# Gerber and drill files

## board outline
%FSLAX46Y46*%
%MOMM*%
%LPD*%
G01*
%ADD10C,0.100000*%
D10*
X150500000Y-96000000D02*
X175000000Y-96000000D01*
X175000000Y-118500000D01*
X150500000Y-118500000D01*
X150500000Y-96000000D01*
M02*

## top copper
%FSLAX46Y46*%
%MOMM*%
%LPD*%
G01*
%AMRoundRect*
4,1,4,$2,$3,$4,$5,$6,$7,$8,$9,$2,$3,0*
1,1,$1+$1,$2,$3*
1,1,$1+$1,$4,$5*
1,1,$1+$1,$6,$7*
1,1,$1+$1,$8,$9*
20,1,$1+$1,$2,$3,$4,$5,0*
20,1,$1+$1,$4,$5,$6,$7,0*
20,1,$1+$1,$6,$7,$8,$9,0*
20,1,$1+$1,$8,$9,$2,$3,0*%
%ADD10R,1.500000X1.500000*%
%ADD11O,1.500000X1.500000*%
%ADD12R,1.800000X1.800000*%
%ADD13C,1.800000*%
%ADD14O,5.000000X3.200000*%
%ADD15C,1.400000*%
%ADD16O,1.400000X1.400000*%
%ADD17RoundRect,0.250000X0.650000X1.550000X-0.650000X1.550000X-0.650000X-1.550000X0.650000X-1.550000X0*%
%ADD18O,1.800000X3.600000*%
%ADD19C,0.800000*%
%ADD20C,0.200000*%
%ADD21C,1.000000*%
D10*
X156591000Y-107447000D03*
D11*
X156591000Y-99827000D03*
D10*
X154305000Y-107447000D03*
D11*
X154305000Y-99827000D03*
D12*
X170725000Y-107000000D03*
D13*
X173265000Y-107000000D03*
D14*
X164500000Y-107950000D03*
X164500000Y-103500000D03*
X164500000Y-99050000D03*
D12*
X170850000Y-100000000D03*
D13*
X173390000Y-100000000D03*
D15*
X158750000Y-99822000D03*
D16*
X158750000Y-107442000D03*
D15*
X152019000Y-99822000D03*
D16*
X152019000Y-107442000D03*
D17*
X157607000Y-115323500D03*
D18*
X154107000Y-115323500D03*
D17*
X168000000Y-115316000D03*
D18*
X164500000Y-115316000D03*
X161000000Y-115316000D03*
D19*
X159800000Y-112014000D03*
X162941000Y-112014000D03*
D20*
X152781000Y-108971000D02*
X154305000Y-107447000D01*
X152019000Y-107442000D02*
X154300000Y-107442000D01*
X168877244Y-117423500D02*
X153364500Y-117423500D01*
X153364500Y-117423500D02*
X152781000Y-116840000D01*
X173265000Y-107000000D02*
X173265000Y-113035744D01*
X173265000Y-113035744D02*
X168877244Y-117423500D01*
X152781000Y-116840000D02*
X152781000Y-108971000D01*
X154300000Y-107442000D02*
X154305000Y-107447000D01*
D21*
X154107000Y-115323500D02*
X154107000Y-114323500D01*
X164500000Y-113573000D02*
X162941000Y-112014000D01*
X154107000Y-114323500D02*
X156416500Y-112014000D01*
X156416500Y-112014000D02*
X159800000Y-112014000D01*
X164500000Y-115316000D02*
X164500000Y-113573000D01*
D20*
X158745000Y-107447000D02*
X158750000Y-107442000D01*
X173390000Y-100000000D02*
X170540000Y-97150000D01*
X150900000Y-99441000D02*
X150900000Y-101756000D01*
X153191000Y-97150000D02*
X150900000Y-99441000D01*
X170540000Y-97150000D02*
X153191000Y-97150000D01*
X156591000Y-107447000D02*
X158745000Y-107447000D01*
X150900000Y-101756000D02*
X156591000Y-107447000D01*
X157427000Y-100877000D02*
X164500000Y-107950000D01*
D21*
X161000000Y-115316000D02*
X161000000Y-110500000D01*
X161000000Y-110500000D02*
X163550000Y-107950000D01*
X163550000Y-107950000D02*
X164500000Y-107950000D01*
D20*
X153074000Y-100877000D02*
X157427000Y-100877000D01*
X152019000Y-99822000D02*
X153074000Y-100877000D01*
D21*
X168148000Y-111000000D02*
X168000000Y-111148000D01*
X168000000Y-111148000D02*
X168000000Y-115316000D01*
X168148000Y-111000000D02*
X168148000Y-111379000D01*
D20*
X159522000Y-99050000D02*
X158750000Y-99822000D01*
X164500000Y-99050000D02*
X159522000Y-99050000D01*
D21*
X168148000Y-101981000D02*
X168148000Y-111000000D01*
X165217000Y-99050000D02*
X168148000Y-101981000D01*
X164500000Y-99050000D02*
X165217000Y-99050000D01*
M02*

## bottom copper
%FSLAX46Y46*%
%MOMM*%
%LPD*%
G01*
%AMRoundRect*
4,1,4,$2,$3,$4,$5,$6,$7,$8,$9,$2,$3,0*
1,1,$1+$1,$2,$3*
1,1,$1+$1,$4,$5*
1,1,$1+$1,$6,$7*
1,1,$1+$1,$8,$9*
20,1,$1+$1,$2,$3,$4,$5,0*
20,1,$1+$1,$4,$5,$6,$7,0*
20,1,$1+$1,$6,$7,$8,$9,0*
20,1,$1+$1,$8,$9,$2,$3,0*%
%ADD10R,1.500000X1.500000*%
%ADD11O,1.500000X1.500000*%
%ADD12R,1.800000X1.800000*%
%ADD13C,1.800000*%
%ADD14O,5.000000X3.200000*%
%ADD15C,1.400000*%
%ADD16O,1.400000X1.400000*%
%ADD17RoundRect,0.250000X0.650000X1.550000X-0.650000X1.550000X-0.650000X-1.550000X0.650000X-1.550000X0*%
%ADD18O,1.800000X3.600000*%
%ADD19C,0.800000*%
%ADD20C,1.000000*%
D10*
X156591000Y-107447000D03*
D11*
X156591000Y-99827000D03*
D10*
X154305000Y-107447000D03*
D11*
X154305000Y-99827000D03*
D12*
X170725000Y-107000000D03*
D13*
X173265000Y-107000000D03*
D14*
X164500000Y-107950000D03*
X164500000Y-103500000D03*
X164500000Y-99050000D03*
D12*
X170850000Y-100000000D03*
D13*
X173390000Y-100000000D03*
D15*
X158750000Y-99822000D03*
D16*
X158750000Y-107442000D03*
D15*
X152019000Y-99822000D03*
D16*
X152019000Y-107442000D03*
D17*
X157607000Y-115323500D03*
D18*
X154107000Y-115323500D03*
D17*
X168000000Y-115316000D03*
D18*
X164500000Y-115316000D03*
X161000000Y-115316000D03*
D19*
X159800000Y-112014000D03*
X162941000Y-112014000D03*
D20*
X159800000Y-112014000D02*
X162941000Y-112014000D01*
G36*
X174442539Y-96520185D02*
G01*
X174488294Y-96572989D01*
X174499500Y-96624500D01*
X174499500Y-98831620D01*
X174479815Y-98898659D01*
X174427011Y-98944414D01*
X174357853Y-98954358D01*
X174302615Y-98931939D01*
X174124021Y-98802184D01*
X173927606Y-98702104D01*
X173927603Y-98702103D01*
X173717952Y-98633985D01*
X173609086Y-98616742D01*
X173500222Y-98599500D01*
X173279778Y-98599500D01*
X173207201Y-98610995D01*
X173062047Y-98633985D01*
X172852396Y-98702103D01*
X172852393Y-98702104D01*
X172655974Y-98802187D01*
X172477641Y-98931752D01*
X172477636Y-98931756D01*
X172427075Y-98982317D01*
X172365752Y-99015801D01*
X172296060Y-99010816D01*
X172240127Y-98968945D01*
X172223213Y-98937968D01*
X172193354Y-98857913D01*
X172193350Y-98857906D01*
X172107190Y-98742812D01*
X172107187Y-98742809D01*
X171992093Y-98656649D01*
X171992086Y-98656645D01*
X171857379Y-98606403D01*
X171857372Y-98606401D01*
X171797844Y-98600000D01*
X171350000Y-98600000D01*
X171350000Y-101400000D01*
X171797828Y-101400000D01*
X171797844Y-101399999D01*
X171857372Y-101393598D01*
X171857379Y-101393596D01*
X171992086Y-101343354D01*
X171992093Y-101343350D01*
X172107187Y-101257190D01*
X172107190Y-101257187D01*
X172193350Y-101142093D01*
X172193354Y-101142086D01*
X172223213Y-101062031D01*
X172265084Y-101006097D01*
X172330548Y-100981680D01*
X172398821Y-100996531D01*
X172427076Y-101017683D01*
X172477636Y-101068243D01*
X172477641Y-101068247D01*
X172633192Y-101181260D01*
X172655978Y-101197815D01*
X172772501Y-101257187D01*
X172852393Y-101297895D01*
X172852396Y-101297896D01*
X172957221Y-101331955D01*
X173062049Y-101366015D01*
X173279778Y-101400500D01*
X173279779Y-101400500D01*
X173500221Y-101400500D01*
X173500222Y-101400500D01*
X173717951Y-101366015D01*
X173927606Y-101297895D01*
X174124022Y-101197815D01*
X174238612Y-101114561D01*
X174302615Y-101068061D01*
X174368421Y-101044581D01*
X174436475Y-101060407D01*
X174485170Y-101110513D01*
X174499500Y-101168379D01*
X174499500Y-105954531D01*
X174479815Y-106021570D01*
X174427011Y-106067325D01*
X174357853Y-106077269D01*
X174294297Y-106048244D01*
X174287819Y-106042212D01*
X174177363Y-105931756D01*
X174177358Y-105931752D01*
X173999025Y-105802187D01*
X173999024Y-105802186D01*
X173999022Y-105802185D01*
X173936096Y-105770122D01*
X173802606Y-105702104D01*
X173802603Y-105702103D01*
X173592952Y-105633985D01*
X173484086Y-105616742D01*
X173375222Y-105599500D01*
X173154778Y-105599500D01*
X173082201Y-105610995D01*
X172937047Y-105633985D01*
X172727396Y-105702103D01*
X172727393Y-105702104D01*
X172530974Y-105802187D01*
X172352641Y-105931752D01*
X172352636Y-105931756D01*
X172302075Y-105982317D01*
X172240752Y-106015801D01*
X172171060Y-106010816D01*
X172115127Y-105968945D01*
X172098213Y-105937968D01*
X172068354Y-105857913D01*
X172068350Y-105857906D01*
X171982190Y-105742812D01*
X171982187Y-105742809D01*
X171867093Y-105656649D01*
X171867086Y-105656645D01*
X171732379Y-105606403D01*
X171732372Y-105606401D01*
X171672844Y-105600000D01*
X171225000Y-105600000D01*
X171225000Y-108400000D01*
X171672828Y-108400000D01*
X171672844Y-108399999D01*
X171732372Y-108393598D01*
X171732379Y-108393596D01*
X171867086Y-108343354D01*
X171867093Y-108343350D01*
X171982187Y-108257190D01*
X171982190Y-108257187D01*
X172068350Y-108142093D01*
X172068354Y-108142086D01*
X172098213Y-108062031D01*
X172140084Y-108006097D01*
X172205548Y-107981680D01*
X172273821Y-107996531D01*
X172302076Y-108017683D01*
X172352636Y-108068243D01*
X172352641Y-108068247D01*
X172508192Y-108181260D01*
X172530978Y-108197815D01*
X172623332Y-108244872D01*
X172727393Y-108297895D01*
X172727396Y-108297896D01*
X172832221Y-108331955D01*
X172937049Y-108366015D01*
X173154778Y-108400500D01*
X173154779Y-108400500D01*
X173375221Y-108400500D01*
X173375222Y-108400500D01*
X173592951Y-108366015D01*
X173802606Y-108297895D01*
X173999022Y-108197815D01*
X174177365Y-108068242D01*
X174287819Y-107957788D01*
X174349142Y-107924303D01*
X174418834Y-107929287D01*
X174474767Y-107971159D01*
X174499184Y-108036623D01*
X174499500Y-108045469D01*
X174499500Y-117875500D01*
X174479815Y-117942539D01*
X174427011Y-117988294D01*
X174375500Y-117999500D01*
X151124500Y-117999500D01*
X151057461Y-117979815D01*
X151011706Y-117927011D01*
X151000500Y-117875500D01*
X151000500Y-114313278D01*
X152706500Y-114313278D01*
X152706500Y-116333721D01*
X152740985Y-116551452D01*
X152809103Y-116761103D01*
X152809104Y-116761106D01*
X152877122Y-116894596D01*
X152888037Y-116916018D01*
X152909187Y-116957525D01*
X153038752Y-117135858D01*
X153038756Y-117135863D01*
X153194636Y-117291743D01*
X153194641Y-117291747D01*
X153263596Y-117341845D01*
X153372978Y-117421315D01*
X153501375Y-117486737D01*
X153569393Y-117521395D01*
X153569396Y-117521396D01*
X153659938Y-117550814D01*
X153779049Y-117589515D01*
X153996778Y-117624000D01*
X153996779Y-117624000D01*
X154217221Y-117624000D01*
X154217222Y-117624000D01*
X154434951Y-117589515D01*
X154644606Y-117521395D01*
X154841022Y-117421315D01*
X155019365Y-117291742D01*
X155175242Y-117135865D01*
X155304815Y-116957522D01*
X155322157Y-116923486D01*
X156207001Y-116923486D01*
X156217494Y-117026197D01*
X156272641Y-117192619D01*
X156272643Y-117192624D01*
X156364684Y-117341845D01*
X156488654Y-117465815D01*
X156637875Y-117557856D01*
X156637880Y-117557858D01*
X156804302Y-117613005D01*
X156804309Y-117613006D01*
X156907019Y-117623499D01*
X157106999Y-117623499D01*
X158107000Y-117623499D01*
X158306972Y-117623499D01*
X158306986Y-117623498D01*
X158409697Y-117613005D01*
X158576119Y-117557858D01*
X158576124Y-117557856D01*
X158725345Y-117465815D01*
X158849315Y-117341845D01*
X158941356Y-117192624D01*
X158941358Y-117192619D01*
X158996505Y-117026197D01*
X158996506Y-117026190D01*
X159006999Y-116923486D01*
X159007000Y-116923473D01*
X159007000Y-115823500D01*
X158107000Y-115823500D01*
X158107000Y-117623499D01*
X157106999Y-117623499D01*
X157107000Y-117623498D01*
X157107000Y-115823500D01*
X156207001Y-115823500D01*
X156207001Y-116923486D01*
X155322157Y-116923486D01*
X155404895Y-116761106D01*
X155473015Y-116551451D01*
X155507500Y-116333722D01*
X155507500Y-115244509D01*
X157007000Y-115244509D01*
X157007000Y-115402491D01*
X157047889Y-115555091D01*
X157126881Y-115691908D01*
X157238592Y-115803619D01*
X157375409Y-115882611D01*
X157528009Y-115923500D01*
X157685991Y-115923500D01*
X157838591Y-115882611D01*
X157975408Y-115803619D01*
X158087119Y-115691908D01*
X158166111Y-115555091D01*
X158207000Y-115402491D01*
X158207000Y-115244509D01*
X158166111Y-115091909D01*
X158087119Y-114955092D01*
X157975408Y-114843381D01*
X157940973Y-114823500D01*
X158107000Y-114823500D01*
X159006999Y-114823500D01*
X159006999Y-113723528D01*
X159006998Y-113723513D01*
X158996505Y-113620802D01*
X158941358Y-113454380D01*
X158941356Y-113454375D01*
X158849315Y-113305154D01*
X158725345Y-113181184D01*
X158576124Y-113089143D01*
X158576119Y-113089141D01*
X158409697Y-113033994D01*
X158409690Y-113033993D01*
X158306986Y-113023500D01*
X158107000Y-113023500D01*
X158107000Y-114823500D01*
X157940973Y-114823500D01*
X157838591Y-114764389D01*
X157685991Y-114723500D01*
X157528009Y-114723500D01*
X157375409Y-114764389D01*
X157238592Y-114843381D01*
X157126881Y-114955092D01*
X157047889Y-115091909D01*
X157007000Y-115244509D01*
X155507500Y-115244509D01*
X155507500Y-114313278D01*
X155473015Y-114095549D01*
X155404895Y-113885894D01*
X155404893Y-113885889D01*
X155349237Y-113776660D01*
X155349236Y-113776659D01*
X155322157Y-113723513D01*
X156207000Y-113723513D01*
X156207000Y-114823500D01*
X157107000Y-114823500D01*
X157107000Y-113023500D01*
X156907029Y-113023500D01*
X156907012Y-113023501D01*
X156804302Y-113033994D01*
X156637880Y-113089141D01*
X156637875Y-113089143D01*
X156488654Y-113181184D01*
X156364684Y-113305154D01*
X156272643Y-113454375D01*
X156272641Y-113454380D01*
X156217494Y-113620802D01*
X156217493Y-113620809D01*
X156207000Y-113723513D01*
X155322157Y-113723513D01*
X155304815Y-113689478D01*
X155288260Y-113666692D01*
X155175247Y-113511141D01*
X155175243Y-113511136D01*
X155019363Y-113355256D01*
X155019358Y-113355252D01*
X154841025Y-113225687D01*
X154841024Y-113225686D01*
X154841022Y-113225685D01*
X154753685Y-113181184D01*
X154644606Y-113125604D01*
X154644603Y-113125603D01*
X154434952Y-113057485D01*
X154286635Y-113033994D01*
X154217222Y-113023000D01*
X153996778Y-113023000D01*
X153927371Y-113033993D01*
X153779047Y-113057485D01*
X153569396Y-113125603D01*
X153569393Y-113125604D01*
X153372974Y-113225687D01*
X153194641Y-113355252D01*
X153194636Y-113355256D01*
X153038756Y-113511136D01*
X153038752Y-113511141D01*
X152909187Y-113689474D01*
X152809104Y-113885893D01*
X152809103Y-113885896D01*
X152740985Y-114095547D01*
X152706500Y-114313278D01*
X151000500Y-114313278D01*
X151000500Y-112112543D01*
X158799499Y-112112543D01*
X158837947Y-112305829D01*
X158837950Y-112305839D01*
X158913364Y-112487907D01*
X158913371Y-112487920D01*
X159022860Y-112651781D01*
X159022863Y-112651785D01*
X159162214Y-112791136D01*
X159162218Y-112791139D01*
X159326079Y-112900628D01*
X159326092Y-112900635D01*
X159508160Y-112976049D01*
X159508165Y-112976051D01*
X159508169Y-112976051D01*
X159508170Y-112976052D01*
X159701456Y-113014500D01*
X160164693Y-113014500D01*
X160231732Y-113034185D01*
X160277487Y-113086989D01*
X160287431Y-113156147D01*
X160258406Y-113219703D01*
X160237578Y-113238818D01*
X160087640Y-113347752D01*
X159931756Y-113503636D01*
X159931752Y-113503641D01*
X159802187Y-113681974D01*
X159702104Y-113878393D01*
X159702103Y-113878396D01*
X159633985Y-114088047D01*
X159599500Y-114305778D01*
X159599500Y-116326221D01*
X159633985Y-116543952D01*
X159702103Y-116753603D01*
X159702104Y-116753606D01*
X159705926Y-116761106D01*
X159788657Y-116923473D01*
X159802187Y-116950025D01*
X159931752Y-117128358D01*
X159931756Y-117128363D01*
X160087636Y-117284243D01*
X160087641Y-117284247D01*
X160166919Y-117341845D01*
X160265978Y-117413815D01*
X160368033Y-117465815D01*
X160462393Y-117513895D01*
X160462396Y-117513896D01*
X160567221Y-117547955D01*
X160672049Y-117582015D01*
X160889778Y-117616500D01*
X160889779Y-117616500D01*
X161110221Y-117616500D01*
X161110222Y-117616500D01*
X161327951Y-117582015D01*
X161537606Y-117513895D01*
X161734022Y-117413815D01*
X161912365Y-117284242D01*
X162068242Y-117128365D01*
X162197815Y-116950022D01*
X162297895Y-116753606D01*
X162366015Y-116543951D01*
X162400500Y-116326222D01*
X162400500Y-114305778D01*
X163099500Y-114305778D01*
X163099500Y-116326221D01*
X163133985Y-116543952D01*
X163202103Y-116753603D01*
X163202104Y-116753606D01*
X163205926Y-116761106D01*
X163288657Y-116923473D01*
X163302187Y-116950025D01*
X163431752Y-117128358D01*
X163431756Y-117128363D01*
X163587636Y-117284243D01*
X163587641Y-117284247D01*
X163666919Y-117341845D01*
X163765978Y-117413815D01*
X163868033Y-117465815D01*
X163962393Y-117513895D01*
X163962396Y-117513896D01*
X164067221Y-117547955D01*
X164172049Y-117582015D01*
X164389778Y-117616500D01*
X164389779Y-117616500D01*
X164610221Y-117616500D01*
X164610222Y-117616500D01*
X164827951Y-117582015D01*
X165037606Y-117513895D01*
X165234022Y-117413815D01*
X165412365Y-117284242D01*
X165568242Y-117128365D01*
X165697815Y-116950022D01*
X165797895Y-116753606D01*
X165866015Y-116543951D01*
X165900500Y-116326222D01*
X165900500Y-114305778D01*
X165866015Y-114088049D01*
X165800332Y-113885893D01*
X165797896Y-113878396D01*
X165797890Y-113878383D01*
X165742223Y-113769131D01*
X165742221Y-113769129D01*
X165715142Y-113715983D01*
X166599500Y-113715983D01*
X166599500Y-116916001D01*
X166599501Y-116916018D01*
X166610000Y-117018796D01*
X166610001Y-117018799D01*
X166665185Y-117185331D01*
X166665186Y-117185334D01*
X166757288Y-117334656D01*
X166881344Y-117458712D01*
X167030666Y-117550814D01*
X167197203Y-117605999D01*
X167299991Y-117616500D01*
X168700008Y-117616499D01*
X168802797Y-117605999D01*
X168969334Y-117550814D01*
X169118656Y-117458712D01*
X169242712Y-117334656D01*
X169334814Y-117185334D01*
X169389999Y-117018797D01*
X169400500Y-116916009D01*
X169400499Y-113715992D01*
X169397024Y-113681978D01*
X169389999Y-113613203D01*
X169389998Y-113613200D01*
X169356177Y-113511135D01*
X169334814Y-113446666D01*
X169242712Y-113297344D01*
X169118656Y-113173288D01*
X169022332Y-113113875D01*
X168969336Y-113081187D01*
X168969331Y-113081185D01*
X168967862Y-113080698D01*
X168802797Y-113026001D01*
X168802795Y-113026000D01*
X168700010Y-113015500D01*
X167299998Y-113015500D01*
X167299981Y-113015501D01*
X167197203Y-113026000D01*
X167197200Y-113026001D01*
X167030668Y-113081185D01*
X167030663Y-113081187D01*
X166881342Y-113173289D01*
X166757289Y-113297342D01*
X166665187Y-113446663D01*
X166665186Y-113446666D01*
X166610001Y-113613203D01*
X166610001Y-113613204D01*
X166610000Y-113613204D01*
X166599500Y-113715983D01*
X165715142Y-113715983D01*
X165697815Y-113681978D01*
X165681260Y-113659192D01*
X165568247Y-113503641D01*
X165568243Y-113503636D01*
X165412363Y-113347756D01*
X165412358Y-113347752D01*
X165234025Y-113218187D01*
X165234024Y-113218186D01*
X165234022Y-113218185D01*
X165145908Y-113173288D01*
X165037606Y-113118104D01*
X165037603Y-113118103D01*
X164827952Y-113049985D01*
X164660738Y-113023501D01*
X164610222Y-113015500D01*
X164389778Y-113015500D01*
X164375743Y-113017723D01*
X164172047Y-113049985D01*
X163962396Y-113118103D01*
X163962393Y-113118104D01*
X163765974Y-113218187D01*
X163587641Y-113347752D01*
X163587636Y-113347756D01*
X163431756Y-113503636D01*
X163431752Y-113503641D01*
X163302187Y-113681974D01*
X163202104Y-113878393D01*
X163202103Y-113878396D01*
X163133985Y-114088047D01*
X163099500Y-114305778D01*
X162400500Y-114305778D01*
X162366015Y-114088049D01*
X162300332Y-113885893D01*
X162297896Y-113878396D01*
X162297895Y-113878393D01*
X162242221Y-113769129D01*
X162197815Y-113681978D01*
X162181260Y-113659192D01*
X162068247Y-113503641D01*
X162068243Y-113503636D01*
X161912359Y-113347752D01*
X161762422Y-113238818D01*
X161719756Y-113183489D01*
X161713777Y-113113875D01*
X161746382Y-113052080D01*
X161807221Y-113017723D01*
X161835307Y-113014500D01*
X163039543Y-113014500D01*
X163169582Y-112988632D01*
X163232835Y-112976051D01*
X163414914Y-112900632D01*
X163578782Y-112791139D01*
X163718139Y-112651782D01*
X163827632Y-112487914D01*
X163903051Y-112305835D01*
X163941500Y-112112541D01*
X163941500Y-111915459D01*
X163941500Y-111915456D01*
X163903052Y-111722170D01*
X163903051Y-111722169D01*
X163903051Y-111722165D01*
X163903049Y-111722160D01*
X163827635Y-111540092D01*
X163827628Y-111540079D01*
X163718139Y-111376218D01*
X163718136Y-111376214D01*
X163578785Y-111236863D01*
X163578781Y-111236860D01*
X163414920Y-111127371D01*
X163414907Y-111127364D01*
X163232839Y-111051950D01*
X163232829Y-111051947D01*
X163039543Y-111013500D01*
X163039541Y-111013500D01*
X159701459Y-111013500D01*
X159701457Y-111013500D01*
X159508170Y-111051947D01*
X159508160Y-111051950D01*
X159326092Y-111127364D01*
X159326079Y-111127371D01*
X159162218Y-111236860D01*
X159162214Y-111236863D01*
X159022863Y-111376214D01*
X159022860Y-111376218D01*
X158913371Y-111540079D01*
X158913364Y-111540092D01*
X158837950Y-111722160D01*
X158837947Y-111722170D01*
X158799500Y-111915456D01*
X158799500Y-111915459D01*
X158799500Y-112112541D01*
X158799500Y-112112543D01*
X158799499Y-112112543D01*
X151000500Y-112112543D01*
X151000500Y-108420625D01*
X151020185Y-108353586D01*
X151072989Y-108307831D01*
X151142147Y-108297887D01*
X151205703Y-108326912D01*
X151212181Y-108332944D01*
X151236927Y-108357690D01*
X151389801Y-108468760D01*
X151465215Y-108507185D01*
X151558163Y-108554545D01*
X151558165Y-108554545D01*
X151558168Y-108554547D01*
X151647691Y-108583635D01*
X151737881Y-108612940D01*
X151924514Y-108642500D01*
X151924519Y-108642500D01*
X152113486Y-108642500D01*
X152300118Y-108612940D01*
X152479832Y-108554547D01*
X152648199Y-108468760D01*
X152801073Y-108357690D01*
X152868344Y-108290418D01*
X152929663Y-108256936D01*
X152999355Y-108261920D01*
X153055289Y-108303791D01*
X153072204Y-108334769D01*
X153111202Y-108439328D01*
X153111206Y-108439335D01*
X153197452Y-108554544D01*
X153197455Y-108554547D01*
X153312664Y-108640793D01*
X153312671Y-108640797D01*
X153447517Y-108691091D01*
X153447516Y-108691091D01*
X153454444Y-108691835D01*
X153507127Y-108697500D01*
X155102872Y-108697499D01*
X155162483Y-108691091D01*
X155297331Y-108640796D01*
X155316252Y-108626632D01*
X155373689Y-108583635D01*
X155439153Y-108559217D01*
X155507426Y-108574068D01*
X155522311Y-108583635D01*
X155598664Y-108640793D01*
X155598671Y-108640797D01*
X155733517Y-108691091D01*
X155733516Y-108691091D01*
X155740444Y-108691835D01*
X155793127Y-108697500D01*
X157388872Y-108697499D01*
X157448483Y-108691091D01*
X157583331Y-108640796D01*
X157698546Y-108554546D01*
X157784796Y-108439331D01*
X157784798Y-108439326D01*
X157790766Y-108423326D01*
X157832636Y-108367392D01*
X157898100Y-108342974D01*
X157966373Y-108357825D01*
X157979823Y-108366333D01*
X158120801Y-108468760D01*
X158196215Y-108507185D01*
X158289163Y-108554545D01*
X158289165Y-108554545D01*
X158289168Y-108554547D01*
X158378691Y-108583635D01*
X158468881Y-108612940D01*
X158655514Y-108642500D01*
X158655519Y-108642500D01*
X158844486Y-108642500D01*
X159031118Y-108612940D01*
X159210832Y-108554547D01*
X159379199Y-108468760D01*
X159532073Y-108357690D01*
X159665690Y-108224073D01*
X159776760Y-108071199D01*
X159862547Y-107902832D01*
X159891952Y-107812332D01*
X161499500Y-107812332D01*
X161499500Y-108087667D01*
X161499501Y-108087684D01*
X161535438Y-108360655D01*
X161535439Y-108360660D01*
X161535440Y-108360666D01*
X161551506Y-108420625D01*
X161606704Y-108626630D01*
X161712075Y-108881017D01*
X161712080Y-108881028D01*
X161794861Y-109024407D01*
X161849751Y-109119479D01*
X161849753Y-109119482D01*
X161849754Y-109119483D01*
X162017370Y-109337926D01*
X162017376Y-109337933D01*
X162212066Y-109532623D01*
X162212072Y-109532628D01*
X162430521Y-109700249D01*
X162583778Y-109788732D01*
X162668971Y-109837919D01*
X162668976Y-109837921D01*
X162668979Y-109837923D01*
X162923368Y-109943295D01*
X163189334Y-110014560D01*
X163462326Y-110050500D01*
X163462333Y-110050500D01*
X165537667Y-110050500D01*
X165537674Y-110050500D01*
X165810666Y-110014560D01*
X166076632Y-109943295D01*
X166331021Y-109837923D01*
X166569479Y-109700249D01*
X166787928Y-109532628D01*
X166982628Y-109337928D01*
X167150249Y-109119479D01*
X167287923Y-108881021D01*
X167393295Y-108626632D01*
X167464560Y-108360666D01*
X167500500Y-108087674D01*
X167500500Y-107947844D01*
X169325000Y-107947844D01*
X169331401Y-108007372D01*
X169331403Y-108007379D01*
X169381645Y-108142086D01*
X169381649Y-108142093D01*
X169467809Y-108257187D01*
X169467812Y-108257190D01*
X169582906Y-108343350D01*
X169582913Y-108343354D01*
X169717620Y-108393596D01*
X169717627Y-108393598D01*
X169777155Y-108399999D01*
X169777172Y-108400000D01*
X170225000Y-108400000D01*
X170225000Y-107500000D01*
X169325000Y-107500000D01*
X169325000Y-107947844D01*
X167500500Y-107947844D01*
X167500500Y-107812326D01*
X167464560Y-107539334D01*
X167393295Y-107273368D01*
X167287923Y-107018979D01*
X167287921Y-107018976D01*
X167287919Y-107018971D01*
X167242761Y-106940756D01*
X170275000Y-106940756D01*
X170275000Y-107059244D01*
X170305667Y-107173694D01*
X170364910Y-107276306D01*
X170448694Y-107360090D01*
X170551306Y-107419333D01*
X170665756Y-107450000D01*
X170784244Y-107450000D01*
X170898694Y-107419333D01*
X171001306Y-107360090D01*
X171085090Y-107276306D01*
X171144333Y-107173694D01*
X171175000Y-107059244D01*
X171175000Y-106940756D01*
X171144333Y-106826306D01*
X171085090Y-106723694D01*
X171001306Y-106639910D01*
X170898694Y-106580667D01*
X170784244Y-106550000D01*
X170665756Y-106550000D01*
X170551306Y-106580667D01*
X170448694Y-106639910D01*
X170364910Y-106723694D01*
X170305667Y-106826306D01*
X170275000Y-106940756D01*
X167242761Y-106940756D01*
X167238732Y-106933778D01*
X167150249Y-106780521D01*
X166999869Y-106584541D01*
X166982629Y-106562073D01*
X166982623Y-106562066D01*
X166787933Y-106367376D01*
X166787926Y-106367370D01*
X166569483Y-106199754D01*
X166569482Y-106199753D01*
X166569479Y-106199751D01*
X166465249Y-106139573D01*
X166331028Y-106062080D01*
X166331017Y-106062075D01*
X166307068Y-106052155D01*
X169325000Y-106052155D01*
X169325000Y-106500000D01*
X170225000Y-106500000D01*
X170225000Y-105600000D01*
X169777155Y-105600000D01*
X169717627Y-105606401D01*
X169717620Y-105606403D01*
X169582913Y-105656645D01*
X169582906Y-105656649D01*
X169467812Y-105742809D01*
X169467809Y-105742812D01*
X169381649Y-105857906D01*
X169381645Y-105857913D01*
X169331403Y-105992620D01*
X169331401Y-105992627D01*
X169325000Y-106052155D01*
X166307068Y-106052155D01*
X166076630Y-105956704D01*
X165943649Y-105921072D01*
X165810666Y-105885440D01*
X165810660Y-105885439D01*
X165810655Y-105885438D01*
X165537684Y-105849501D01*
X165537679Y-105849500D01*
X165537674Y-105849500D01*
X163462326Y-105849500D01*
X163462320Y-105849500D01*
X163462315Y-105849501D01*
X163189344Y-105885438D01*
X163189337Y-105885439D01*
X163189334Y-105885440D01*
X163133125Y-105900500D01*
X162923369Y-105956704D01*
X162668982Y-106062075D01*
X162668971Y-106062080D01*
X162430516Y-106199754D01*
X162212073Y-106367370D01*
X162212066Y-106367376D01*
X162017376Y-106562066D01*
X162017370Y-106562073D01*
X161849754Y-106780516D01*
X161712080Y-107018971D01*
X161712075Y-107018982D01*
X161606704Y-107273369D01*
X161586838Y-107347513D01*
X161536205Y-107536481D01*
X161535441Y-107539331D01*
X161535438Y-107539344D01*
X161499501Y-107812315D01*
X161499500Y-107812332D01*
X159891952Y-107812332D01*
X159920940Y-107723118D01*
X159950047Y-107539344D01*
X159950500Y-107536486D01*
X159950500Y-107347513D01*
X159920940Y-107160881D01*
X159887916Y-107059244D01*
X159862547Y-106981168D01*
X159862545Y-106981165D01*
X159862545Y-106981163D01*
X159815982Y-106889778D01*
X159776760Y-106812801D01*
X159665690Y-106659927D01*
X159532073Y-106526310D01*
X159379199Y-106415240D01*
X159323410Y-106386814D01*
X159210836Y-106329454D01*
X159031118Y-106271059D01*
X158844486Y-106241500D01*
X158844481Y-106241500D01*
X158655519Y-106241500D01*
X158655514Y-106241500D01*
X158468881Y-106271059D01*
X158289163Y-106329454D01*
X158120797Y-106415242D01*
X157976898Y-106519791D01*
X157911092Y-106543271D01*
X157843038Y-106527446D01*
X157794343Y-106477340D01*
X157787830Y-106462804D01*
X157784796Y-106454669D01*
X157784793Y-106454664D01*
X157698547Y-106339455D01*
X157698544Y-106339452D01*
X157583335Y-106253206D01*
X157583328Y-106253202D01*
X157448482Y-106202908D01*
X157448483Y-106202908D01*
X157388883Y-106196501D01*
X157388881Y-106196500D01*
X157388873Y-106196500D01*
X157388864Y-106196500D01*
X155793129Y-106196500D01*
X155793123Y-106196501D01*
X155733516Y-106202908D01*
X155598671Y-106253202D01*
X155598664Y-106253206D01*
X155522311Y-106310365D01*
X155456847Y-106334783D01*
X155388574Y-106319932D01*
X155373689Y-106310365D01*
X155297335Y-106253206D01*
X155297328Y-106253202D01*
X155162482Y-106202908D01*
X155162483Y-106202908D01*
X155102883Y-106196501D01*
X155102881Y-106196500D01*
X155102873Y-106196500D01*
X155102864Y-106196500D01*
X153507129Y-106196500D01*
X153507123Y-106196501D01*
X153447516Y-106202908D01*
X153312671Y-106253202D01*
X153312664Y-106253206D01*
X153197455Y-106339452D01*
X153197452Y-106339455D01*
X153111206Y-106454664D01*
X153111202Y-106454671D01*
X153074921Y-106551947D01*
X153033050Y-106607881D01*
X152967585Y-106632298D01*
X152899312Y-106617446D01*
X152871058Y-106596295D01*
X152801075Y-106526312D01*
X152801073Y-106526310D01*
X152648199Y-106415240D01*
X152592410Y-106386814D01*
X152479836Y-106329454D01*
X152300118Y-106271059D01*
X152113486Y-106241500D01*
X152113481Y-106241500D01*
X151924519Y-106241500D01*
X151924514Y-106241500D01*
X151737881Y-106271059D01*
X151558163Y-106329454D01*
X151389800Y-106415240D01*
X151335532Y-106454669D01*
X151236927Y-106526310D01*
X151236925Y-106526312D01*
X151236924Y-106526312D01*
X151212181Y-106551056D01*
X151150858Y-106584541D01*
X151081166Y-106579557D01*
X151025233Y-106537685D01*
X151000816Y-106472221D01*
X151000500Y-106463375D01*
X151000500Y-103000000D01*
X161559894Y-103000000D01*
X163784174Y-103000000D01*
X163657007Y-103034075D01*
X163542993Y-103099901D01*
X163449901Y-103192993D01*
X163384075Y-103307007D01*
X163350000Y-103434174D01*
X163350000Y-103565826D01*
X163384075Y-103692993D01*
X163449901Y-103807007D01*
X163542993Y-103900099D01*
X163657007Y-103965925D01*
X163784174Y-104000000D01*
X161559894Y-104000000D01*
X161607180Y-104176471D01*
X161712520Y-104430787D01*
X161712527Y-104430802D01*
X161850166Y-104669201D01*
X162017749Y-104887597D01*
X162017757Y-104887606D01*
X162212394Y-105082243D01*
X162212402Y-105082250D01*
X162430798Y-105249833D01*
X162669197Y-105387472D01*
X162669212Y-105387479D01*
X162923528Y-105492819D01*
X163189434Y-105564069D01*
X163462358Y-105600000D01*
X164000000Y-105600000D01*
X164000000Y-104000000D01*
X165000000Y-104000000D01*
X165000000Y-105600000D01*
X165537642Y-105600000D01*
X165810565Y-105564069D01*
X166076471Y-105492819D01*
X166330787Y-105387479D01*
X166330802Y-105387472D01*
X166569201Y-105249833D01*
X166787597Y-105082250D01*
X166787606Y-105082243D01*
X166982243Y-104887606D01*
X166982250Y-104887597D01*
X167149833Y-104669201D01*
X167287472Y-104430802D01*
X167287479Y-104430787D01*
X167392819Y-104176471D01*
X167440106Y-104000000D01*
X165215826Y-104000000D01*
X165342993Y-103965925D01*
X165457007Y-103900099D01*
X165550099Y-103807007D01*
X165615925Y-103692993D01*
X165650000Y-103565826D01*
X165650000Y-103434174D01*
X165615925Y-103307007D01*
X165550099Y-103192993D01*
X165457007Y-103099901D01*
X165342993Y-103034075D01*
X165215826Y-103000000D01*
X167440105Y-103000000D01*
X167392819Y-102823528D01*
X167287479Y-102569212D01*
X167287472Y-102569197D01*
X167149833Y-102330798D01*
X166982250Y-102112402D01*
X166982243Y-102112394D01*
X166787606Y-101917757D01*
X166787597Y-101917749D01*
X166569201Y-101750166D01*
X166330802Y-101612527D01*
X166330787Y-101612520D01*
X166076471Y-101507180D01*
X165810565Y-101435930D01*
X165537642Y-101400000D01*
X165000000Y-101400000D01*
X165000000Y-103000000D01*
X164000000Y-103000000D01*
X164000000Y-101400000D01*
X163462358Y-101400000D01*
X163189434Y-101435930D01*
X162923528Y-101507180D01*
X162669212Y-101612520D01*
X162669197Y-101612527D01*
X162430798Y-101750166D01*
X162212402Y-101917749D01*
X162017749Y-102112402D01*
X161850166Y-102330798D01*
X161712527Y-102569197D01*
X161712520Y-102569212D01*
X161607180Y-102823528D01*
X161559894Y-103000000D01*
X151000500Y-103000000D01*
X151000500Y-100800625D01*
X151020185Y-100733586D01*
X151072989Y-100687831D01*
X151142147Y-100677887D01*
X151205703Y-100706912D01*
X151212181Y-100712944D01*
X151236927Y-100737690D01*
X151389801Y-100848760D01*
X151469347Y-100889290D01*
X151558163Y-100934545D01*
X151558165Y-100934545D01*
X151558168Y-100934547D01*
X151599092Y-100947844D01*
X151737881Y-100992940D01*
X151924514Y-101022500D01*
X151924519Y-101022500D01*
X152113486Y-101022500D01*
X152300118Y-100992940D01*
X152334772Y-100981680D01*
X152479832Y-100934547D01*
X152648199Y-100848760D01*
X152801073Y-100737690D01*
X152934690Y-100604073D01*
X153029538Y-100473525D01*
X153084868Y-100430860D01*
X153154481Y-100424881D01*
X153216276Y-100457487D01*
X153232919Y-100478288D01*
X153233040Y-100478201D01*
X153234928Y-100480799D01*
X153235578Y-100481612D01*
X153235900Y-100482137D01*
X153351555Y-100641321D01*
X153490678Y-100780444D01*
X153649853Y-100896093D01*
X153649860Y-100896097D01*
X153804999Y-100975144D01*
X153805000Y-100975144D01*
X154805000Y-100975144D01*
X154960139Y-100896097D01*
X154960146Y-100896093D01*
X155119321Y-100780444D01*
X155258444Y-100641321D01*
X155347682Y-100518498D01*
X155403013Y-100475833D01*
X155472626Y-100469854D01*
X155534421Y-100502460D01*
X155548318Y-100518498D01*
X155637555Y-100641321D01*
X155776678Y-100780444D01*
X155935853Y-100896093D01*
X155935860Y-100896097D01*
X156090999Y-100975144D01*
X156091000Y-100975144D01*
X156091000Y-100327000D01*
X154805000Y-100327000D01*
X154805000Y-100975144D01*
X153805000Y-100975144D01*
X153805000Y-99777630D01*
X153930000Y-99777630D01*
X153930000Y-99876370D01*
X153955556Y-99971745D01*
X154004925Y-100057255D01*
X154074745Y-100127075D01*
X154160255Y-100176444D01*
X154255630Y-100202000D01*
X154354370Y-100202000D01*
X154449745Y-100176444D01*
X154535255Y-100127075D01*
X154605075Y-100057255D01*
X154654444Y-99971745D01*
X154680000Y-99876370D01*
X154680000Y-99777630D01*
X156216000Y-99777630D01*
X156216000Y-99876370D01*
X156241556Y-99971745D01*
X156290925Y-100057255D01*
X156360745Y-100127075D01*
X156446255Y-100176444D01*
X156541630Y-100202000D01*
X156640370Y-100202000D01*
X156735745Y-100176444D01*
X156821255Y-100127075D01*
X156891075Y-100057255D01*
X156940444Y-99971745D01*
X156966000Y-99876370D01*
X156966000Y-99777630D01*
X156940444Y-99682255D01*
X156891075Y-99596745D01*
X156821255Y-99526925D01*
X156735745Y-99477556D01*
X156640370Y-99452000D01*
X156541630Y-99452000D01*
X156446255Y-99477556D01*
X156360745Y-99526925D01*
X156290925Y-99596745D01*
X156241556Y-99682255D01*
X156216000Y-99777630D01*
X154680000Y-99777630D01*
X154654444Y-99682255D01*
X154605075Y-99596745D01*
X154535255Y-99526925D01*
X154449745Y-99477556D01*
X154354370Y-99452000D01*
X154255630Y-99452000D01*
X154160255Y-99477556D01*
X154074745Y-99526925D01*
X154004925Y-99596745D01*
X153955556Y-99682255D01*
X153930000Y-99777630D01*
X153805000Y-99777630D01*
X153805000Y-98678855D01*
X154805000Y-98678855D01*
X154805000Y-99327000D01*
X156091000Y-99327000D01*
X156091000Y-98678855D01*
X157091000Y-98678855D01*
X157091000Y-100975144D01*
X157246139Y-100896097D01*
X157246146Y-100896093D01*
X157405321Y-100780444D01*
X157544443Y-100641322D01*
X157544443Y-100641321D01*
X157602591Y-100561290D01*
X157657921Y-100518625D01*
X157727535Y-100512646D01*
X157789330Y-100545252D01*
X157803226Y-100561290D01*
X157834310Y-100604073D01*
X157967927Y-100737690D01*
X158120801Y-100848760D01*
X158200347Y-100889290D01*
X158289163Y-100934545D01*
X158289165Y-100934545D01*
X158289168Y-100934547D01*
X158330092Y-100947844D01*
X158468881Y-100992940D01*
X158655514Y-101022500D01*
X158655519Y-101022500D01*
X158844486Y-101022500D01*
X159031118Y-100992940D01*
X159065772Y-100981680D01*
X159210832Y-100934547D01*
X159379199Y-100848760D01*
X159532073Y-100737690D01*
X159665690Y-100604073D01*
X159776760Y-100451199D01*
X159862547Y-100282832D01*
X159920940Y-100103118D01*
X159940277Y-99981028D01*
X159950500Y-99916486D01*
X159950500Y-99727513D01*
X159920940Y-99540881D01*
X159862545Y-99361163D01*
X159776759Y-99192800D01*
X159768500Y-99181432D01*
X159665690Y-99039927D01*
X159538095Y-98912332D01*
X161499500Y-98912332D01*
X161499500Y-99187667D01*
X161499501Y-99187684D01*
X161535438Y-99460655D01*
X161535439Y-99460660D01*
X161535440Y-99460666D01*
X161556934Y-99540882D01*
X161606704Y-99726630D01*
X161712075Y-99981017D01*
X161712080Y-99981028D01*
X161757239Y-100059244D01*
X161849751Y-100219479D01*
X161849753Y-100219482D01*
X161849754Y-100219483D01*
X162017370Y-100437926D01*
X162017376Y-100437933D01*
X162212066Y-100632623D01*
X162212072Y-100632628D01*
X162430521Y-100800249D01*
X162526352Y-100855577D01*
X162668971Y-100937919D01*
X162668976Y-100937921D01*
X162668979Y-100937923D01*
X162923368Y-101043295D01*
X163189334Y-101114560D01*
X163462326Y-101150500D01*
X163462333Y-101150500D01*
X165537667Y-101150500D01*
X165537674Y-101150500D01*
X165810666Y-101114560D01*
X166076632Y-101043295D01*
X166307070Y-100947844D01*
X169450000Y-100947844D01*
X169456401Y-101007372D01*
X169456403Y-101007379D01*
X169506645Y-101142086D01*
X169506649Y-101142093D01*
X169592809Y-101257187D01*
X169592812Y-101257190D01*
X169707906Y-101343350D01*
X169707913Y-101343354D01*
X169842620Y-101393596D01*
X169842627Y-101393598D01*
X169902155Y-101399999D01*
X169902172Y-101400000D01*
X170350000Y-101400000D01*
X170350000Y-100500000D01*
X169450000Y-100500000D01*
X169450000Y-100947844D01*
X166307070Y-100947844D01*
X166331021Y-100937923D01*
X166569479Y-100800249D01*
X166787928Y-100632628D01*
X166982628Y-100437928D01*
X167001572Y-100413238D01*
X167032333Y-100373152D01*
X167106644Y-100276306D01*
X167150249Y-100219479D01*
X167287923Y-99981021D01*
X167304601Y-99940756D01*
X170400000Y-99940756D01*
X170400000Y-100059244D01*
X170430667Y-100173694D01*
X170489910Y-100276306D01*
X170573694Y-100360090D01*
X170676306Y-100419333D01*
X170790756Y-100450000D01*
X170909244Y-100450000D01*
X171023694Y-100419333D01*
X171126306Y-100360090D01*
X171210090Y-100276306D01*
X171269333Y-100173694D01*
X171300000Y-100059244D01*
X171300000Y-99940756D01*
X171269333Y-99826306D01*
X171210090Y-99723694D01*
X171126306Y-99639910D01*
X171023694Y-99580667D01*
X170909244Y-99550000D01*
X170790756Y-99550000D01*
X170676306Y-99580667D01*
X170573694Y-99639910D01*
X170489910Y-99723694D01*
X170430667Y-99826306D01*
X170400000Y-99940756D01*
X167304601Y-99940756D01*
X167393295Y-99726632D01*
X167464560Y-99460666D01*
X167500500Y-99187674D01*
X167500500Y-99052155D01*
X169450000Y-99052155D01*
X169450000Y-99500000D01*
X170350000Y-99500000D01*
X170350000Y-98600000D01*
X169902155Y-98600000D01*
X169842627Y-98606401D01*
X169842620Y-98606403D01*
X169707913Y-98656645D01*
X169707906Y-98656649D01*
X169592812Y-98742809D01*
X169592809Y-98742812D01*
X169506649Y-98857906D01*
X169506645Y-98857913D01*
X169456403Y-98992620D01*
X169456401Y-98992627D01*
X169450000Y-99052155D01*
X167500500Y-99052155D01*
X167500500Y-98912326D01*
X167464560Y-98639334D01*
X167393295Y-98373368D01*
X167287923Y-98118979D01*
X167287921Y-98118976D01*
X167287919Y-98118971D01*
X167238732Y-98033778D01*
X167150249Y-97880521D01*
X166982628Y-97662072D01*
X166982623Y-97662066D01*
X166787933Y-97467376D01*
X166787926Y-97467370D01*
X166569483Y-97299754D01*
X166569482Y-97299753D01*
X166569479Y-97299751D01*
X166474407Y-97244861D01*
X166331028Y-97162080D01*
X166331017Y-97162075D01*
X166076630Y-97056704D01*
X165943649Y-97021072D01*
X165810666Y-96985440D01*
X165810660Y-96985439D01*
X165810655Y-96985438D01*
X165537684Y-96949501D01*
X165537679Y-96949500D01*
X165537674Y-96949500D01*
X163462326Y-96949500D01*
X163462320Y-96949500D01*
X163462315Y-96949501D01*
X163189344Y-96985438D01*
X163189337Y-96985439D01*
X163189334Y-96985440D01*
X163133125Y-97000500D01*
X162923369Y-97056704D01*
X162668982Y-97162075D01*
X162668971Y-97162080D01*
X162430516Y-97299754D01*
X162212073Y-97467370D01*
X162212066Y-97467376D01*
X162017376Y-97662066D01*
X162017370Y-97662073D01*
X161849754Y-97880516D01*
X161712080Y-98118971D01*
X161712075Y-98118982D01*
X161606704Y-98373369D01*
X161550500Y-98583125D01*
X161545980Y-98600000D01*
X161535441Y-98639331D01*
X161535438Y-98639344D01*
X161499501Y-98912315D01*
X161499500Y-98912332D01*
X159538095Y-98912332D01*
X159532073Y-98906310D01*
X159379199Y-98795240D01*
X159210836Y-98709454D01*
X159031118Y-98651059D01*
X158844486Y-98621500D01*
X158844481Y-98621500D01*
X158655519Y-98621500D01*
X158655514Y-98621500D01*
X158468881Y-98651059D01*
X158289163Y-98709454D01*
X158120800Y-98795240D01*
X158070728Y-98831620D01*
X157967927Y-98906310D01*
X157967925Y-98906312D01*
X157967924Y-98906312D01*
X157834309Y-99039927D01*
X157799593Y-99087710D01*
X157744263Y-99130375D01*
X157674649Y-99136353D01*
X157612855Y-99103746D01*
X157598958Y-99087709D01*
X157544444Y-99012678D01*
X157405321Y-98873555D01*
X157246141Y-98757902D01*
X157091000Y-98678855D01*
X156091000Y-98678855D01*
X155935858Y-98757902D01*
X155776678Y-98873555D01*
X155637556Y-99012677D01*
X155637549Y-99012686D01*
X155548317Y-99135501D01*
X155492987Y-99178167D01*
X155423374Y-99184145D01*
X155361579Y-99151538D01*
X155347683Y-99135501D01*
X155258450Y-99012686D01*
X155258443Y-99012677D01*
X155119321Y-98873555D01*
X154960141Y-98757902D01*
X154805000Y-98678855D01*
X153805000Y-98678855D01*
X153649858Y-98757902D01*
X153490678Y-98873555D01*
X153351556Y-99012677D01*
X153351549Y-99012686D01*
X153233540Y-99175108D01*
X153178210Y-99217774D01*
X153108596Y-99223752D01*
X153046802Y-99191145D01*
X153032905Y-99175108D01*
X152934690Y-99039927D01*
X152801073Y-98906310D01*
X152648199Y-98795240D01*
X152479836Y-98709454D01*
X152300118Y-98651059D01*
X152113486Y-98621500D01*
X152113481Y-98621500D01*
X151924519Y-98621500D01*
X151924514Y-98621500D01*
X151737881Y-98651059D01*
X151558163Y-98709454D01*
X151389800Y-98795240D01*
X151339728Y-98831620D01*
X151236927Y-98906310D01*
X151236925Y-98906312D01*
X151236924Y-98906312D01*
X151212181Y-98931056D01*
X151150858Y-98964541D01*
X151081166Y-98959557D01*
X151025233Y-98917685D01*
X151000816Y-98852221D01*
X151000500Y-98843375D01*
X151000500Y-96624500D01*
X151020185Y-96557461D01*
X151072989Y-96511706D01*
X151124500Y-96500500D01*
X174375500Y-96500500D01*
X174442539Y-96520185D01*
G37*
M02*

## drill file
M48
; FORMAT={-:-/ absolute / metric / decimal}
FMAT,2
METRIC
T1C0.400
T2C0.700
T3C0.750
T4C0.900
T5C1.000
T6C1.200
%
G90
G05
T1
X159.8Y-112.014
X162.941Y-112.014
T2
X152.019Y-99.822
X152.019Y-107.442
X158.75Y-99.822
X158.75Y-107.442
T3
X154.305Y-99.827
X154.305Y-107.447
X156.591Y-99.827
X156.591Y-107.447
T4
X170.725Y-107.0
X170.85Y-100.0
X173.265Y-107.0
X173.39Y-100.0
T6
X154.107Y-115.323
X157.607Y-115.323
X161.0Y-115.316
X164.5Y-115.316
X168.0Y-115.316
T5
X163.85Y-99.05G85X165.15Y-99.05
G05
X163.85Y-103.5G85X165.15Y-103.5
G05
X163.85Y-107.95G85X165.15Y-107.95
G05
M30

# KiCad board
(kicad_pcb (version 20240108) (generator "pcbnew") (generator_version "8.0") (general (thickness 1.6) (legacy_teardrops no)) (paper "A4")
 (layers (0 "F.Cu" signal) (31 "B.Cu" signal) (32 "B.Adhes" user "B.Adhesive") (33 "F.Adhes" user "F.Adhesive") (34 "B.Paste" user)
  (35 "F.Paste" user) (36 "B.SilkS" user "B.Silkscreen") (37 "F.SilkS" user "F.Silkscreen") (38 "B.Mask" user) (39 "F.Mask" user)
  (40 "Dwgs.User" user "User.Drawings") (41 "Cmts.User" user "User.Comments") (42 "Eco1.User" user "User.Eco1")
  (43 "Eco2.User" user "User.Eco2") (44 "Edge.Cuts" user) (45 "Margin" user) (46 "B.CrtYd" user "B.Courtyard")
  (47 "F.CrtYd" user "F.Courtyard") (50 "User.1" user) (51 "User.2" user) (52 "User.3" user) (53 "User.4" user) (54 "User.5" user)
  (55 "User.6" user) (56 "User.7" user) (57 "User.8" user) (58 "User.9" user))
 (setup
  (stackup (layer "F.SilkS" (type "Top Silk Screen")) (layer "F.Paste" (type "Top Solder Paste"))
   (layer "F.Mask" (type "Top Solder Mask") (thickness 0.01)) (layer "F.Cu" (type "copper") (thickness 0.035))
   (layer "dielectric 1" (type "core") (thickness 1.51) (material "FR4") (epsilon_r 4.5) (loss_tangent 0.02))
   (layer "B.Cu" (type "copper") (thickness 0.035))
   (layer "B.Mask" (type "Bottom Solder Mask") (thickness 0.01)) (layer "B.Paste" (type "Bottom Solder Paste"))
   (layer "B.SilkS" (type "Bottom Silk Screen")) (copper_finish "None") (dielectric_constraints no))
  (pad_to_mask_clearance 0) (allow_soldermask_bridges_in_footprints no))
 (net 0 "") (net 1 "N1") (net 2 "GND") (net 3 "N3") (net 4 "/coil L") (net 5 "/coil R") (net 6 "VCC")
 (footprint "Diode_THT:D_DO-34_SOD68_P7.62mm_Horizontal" (layer "F.Cu") (at 156.591 107.447 90)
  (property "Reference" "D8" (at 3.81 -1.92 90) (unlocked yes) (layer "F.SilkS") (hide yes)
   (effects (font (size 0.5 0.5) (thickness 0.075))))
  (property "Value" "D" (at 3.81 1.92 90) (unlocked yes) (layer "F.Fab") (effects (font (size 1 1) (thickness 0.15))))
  (pad "1" thru_hole rect (at 0 0 90) (size 1.5 1.5) (drill 0.75) (layers "*.Cu" "*.Mask") (remove_unused_layers no) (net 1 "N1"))
  (pad "2" thru_hole oval (at 7.62 0 90) (size 1.5 1.5) (drill 0.75) (layers "*.Cu" "*.Mask") (remove_unused_layers no) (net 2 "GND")))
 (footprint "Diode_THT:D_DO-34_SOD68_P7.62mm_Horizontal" (layer "F.Cu") (at 154.305 107.447 90)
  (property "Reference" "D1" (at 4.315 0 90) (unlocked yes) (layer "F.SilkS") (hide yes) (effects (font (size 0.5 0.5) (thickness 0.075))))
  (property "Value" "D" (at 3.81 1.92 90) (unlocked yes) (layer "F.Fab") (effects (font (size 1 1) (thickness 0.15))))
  (pad "1" thru_hole rect (at 0 0 90) (size 1.5 1.5) (drill 0.75) (layers "*.Cu" "*.Mask") (remove_unused_layers no) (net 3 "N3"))
  (pad "2" thru_hole oval (at 7.62 0 90) (size 1.5 1.5) (drill 0.75) (layers "*.Cu" "*.Mask") (remove_unused_layers no) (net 2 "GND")))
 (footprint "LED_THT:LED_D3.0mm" (layer "F.Cu") (at 170.725 107)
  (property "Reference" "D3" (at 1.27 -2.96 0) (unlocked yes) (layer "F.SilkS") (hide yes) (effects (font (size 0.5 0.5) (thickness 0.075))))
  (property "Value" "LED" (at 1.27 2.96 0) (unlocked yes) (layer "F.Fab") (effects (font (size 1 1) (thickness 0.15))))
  (pad "1" thru_hole rect (at 0 0) (size 1.8 1.8) (drill 0.9) (layers "*.Cu" "*.Mask") (remove_unused_layers no) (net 2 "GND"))
  (pad "2" thru_hole circle (at 2.54 0) (size 1.8 1.8) (drill 0.9) (layers "*.Cu" "*.Mask") (remove_unused_layers no) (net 3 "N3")))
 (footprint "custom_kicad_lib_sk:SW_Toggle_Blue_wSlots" (layer "F.Cu") (at 164.5 103.5 90)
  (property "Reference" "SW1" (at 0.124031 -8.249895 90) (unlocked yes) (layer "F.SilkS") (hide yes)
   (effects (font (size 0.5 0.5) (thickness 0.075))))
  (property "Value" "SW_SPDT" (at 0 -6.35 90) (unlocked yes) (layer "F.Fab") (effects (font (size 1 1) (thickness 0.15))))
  (pad "1" thru_hole oval (at -4.45 0 90) (size 3.2 5) (drill oval 1 2.3) (layers "*.Cu" "*.Mask") (remove_unused_layers no)
   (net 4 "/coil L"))
  (pad "2" thru_hole oval (at 0 0 90) (size 3.2 5) (drill oval 1 2.3) (layers "*.Cu" "*.Mask") (remove_unused_layers no) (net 2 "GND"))
  (pad "3" thru_hole oval (at 4.45 0 90) (size 3.2 5) (drill oval 1 2.3) (layers "*.Cu" "*.Mask") (remove_unused_layers no)
   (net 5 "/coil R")))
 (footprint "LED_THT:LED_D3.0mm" (layer "F.Cu") (at 170.85 100)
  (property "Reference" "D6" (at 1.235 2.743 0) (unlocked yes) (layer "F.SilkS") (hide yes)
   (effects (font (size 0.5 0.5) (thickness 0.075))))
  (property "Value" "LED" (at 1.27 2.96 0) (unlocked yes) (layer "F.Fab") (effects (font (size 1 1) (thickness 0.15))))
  (pad "1" thru_hole rect (at 0 0) (size 1.8 1.8) (drill 0.9) (layers "*.Cu" "*.Mask") (remove_unused_layers no) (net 2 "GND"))
  (pad "2" thru_hole circle (at 2.54 0) (size 1.8 1.8) (drill 0.9) (layers "*.Cu" "*.Mask") (remove_unused_layers no) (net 1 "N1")))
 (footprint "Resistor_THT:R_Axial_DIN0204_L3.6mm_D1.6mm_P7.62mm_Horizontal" (layer "F.Cu") (at 158.75 99.822 -90)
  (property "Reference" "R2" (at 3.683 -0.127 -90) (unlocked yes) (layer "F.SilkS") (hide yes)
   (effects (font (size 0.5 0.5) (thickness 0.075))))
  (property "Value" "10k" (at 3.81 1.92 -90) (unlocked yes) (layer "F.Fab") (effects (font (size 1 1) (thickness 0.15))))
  (pad "1" thru_hole circle (at 0 0 270) (size 1.4 1.4) (drill 0.7) (layers "*.Cu" "*.Mask") (remove_unused_layers no) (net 5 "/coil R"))
  (pad "2" thru_hole oval (at 7.62 0 270) (size 1.4 1.4) (drill 0.7) (layers "*.Cu" "*.Mask") (remove_unused_layers no) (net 1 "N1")))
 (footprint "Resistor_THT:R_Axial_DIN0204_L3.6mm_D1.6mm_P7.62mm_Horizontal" (layer "F.Cu") (at 152.019 99.822 -90)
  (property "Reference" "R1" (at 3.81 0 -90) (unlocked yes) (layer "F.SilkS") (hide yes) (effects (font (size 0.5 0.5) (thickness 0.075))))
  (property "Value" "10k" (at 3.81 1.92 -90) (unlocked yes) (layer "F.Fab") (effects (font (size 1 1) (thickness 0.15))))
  (pad "1" thru_hole circle (at 0 0 270) (size 1.4 1.4) (drill 0.7) (layers "*.Cu" "*.Mask") (remove_unused_layers no) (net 4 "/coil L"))
  (pad "2" thru_hole oval (at 7.62 0 270) (size 1.4 1.4) (drill 0.7) (layers "*.Cu" "*.Mask") (remove_unused_layers no) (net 3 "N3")))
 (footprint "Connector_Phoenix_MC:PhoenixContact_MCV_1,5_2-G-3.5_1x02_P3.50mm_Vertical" (layer "B.Cu") (at 157.607 115.3235 180)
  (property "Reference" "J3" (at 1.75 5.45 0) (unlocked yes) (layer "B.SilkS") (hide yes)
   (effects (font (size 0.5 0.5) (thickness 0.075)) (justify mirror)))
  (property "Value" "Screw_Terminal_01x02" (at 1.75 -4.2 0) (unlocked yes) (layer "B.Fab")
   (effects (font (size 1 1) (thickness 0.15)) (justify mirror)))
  (pad "1" thru_hole roundrect (at 0 0 180) (size 1.8 3.6) (drill 1.2) (layers "*.Cu" "*.Mask") (remove_unused_layers no)
   (roundrect_rratio 0.138889) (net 2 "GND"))
  (pad "2" thru_hole oval (at 3.5 0 180) (size 1.8 3.6) (drill 1.2) (layers "*.Cu" "*.Mask") (remove_unused_layers no) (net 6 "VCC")))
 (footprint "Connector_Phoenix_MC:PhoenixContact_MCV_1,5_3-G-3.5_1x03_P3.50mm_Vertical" (layer "B.Cu") (at 168 115.316 180)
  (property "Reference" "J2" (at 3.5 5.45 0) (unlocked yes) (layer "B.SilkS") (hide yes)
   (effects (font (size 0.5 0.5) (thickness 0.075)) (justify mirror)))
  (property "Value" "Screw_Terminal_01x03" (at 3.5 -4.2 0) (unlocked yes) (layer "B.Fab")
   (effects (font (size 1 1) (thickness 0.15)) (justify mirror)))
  (pad "1" thru_hole roundrect (at 0 0 180) (size 1.8 3.6) (drill 1.2) (layers "*.Cu" "*.Mask") (remove_unused_layers no)
   (roundrect_rratio 0.138889) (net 5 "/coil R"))
  (pad "2" thru_hole oval (at 3.5 0 180) (size 1.8 3.6) (drill 1.2) (layers "*.Cu" "*.Mask") (remove_unused_layers no) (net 6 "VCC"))
  (pad "3" thru_hole oval (at 7 0 180) (size 1.8 3.6) (drill 1.2) (layers "*.Cu" "*.Mask") (remove_unused_layers no) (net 4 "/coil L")))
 (gr_rect (start 150.5 96) (end 175 118.5) (stroke (width 0.1) (type default)) (fill none) (layer "Edge.Cuts"))
 (segment (start 152.781 108.971) (end 154.305 107.447) (width 0.2) (layer "F.Cu") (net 3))
 (segment (start 152.019 107.442) (end 154.3 107.442) (width 0.2) (layer "F.Cu") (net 3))
 (segment (start 168.877244 117.4235) (end 153.3645 117.4235) (width 0.2) (layer "F.Cu") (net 3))
 (segment (start 153.3645 117.4235) (end 152.781 116.84) (width 0.2) (layer "F.Cu") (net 3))
 (segment (start 173.265 107) (end 173.265 113.035744) (width 0.2) (layer "F.Cu") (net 3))
 (segment (start 173.265 113.035744) (end 168.877244 117.4235) (width 0.2) (layer "F.Cu") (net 3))
 (segment (start 152.781 116.84) (end 152.781 108.971) (width 0.2) (layer "F.Cu") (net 3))
 (segment (start 154.3 107.442) (end 154.305 107.447) (width 0.2) (layer "F.Cu") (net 3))
 (segment (start 154.107 115.3235) (end 154.107 114.3235) (width 1) (layer "F.Cu") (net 6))
 (segment (start 164.5 113.573) (end 162.941 112.014) (width 1) (layer "F.Cu") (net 6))
 (segment (start 154.107 114.3235) (end 156.4165 112.014) (width 1) (layer "F.Cu") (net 6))
 (segment (start 156.4165 112.014) (end 159.8 112.014) (width 1) (layer "F.Cu") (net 6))
 (segment (start 164.5 115.316) (end 164.5 113.573) (width 1) (layer "F.Cu") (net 6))
 (via (at 159.8 112.014) (size 0.8) (drill 0.4) (layers "F.Cu" "B.Cu") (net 6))
 (via (at 162.941 112.014) (size 0.8) (drill 0.4) (layers "F.Cu" "B.Cu") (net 6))
 (segment (start 159.8 112.014) (end 162.941 112.014) (width 1) (layer "B.Cu") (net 6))
 (segment (start 158.745 107.447) (end 158.75 107.442) (width 0.2) (layer "F.Cu") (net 1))
 (segment (start 173.39 100) (end 170.54 97.15) (width 0.2) (layer "F.Cu") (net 1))
 (segment (start 150.9 99.441) (end 150.9 101.756) (width 0.2) (layer "F.Cu") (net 1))
 (segment (start 153.191 97.15) (end 150.9 99.441) (width 0.2) (layer "F.Cu") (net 1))
 (segment (start 170.54 97.15) (end 153.191 97.15) (width 0.2) (layer "F.Cu") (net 1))
 (segment (start 156.591 107.447) (end 158.745 107.447) (width 0.2) (layer "F.Cu") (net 1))
 (segment (start 150.9 101.756) (end 156.591 107.447) (width 0.2) (layer "F.Cu") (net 1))
 (segment (start 157.427 100.877) (end 164.5 107.95) (width 0.2) (layer "F.Cu") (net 4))
 (segment (start 161 115.316) (end 161 110.5) (width 1) (layer "F.Cu") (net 4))
 (segment (start 161 110.5) (end 163.55 107.95) (width 1) (layer "F.Cu") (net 4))
 (segment (start 163.55 107.95) (end 164.5 107.95) (width 1) (layer "F.Cu") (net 4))
 (segment (start 153.074 100.877) (end 157.427 100.877) (width 0.2) (layer "F.Cu") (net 4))
 (segment (start 152.019 99.822) (end 153.074 100.877) (width 0.2) (layer "F.Cu") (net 4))
 (segment (start 168.148 111) (end 168 111.148) (width 1) (layer "F.Cu") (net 5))
 (segment (start 168 111.148) (end 168 115.316) (width 1) (layer "F.Cu") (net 5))
 (segment (start 168.148 111) (end 168.148 111.379) (width 1) (layer "F.Cu") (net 5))
 (segment (start 159.522 99.05) (end 158.75 99.822) (width 0.2) (layer "F.Cu") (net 5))
 (segment (start 164.5 99.05) (end 159.522 99.05) (width 0.2) (layer "F.Cu") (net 5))
 (segment (start 168.148 101.981) (end 168.148 111) (width 1) (layer "F.Cu") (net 5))
 (segment (start 165.217 99.05) (end 168.148 101.981) (width 1) (layer "F.Cu") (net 5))
 (segment (start 164.5 99.05) (end 165.217 99.05) (width 1) (layer "F.Cu") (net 5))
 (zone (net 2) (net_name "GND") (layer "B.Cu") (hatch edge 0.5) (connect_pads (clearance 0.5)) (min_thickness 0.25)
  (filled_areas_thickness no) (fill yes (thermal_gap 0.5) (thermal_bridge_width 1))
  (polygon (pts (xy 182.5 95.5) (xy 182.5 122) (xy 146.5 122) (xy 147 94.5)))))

